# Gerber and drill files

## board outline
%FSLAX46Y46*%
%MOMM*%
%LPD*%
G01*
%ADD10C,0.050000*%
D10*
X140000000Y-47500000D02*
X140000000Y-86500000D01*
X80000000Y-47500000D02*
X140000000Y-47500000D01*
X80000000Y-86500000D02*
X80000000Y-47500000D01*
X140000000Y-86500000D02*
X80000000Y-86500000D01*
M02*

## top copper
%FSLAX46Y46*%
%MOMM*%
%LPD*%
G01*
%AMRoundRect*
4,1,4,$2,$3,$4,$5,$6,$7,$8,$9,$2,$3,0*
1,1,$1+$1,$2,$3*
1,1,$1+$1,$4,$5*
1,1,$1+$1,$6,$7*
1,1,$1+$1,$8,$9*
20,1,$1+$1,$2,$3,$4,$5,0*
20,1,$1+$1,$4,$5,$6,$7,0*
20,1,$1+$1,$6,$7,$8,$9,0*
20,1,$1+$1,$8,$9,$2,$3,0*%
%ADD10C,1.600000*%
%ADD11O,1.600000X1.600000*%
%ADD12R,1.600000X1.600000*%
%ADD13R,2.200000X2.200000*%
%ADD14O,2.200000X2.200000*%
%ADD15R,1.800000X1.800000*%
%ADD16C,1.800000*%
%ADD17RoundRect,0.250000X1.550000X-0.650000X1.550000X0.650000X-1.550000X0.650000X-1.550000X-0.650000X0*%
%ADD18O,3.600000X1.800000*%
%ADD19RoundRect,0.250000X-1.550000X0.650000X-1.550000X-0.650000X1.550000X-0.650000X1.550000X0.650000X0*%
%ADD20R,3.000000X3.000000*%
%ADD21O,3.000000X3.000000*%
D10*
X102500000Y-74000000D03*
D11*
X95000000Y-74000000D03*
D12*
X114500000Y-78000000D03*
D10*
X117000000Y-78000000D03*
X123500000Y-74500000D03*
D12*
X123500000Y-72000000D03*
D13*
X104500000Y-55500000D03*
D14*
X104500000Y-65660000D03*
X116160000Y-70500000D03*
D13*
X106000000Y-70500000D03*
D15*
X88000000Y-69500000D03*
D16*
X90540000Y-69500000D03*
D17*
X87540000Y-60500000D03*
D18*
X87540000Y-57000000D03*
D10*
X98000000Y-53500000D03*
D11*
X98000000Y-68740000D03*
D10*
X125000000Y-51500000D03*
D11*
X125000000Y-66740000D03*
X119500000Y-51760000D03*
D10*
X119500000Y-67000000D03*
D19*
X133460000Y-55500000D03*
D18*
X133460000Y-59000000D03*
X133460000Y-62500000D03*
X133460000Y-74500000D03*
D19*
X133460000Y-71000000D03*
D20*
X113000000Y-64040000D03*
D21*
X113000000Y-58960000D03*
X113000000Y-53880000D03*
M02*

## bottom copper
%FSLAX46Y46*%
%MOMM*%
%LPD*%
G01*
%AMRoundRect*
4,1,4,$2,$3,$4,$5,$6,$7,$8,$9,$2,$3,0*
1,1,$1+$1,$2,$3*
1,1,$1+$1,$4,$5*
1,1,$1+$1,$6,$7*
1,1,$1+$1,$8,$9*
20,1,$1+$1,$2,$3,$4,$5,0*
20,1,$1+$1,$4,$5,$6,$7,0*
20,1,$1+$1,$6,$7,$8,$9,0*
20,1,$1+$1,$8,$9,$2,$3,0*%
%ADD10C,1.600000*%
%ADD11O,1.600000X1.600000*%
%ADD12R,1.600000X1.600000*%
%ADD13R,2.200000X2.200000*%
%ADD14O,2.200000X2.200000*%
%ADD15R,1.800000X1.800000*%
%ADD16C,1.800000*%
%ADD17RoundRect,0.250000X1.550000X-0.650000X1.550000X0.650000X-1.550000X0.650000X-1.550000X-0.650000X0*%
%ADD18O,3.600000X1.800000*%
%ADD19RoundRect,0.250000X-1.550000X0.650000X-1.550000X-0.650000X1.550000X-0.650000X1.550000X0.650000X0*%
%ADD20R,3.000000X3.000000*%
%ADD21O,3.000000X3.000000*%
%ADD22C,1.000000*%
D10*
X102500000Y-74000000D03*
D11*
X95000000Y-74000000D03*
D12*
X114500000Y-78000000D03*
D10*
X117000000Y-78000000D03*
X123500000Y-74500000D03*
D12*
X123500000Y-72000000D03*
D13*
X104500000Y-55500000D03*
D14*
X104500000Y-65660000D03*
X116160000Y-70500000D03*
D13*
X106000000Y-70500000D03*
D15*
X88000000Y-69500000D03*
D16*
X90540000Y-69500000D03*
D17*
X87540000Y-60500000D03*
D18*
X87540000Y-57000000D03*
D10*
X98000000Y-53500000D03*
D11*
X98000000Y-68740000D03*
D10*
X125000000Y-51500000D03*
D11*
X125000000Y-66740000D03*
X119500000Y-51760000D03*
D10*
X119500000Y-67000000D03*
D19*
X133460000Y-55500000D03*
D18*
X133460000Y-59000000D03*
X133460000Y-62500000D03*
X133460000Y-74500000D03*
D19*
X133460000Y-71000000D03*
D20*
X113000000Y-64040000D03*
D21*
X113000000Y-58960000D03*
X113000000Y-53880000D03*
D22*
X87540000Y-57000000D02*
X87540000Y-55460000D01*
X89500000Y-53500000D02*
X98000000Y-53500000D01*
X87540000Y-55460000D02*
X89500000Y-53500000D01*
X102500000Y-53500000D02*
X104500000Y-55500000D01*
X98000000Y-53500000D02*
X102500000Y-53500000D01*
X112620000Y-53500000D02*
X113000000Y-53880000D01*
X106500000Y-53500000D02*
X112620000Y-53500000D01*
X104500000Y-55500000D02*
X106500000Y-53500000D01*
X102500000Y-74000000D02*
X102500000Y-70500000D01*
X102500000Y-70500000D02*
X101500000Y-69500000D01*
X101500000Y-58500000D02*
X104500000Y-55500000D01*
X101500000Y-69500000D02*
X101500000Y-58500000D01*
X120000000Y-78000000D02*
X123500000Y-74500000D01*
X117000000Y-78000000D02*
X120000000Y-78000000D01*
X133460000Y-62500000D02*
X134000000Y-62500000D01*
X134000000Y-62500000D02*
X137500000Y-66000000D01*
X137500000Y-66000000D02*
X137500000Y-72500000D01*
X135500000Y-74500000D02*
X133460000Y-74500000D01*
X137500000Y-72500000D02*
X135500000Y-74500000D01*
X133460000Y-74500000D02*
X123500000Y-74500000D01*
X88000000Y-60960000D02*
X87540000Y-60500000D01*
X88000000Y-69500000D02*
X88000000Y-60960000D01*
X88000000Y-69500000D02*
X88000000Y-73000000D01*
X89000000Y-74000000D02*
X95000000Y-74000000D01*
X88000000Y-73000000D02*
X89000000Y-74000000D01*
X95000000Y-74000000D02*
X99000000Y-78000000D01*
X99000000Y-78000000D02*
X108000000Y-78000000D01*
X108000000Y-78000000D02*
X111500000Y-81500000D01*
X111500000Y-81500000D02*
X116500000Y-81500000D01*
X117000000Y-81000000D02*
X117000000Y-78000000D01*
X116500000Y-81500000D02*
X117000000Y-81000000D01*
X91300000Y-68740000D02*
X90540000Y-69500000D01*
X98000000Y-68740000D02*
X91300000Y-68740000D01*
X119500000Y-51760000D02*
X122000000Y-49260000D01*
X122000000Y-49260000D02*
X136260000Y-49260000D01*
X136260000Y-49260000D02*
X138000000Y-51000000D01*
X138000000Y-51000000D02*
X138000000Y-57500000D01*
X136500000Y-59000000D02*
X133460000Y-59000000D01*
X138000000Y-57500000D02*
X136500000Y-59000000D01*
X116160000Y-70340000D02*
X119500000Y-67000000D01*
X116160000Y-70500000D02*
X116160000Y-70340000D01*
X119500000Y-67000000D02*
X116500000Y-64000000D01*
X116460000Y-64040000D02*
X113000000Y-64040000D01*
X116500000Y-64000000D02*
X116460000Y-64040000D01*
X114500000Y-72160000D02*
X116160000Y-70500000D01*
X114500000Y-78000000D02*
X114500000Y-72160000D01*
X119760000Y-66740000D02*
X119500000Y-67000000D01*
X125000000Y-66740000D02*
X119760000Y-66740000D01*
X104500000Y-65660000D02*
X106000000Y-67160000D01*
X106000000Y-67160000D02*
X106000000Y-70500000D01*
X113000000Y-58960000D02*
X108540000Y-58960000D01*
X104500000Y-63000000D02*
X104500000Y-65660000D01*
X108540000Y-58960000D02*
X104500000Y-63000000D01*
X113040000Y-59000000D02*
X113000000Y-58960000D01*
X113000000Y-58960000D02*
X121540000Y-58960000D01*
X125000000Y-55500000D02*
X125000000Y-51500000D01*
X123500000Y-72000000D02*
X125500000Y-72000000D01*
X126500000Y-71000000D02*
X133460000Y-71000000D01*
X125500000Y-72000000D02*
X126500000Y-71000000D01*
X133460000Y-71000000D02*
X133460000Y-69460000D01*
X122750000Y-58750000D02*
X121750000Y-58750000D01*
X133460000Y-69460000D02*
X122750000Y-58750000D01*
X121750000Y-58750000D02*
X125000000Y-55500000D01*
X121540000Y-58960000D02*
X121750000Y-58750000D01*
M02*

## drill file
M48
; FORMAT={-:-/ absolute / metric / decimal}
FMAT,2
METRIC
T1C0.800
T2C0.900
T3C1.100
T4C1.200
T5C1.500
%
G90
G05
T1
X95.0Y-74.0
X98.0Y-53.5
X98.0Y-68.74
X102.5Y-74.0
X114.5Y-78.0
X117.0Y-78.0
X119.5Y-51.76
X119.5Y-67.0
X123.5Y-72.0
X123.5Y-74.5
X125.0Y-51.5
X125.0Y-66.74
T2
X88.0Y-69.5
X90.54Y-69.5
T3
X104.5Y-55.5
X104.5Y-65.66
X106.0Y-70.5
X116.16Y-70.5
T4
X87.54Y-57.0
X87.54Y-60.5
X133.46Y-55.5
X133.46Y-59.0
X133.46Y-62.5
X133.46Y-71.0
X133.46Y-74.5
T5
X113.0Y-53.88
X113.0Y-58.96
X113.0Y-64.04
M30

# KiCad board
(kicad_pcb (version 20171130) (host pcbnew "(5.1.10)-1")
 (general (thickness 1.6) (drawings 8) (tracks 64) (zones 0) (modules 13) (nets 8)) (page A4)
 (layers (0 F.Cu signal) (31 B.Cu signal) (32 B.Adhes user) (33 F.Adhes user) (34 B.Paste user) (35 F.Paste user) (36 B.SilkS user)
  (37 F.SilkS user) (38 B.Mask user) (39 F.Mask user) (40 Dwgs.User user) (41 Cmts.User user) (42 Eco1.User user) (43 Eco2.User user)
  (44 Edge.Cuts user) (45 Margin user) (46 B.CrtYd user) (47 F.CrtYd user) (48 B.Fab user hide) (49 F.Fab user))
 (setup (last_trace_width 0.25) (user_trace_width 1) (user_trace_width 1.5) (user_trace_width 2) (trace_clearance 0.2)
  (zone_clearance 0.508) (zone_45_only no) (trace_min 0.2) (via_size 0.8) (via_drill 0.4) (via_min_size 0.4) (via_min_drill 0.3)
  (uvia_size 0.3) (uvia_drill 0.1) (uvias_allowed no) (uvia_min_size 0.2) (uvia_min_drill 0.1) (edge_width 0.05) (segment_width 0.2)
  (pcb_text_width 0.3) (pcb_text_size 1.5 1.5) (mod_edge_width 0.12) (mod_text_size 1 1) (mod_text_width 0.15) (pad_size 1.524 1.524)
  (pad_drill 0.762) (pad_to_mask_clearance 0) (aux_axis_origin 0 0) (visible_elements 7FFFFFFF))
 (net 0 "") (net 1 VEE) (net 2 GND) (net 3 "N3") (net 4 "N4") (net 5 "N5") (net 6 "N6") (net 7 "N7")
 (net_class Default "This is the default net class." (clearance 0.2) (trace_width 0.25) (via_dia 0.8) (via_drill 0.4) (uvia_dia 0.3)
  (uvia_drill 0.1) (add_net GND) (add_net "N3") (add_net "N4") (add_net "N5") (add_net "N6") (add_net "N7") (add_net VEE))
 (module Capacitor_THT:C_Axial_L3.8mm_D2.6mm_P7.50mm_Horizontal (layer F.Cu) (at 102.5 74 180)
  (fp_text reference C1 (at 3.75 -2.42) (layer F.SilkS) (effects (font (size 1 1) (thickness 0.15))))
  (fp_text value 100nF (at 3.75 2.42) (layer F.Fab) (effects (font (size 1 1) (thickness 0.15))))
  (pad 1 thru_hole circle (at 0 0 180) (size 1.6 1.6) (drill 0.8) (layers *.Cu *.Mask) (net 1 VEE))
  (pad 2 thru_hole oval (at 7.5 0 180) (size 1.6 1.6) (drill 0.8) (layers *.Cu *.Mask) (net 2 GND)))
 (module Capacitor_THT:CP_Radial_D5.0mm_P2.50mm (layer F.Cu) (at 114.5 78)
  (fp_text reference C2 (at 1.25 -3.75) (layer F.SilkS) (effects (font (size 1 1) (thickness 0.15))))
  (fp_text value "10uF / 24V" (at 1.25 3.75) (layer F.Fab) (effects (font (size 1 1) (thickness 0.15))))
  (pad 1 thru_hole rect (at 0 0) (size 1.6 1.6) (drill 0.8) (layers *.Cu *.Mask) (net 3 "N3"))
  (pad 2 thru_hole circle (at 2.5 0) (size 1.6 1.6) (drill 0.8) (layers *.Cu *.Mask) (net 2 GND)))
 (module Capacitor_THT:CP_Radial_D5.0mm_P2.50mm (layer F.Cu) (at 123.5 72 270)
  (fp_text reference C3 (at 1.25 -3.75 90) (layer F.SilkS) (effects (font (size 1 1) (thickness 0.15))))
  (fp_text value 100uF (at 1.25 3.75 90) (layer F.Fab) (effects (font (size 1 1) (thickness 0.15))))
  (pad 2 thru_hole circle (at 2.5 0 270) (size 1.6 1.6) (drill 0.8) (layers *.Cu *.Mask) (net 2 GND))
  (pad 1 thru_hole rect (at 0 0 270) (size 1.6 1.6) (drill 0.8) (layers *.Cu *.Mask) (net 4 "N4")))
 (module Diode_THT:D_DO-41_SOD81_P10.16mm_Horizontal (layer F.Cu) (at 104.5 55.5 270)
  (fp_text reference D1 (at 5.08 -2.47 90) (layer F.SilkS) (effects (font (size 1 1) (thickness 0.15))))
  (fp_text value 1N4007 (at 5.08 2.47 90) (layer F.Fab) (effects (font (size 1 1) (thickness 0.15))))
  (pad 1 thru_hole rect (at 0 0 270) (size 2.2 2.2) (drill 1.1) (layers *.Cu *.Mask) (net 1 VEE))
  (pad 2 thru_hole oval (at 10.16 0 270) (size 2.2 2.2) (drill 1.1) (layers *.Cu *.Mask) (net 4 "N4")))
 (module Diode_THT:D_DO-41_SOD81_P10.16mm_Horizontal (layer F.Cu) (at 106 70.5)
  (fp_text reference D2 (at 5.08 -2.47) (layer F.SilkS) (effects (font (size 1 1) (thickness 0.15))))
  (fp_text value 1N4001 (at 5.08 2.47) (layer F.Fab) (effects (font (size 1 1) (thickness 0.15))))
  (pad 2 thru_hole oval (at 10.16 0) (size 2.2 2.2) (drill 1.1) (layers *.Cu *.Mask) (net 3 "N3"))
  (pad 1 thru_hole rect (at 0 0) (size 2.2 2.2) (drill 1.1) (layers *.Cu *.Mask) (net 4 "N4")))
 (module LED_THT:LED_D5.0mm (layer F.Cu) (at 88 69.5)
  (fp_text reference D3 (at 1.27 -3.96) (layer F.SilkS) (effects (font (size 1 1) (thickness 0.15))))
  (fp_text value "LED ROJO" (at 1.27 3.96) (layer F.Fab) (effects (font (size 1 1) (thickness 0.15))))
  (pad 1 thru_hole rect (at 0 0) (size 1.8 1.8) (drill 0.9) (layers *.Cu *.Mask) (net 2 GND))
  (pad 2 thru_hole circle (at 2.54 0) (size 1.8 1.8) (drill 0.9) (layers *.Cu *.Mask) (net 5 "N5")))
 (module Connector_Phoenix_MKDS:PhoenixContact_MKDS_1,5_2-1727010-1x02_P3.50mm (layer F.Cu) (at 85 60.5 90)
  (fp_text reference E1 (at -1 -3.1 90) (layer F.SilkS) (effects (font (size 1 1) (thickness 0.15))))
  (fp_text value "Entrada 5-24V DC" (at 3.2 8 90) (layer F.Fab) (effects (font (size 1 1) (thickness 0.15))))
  (pad 1 thru_hole roundrect (at 0 2.54 90) (size 1.8 3.6) (drill 1.2) (layers *.Cu *.Mask) (roundrect_rratio 0.138889) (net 2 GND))
  (pad 2 thru_hole oval (at 3.5 2.54 90) (size 1.8 3.6) (drill 1.2) (layers *.Cu *.Mask) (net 1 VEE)))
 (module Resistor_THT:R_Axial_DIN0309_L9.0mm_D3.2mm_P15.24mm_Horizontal (layer F.Cu) (at 98 53.5 270)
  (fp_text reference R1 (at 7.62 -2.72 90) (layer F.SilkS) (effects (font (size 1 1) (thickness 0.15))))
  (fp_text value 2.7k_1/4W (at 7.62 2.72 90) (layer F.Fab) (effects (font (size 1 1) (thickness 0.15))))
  (pad 1 thru_hole circle (at 0 0 270) (size 1.6 1.6) (drill 0.8) (layers *.Cu *.Mask) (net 1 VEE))
  (pad 2 thru_hole oval (at 15.24 0 270) (size 1.6 1.6) (drill 0.8) (layers *.Cu *.Mask) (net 5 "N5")))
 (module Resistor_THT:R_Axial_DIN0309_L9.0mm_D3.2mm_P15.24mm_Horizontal (layer F.Cu) (at 125 51.5 270)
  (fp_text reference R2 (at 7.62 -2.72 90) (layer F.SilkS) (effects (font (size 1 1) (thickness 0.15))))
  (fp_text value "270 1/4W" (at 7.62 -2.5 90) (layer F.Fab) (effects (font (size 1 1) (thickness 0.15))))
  (pad 1 thru_hole circle (at 0 0 270) (size 1.6 1.6) (drill 0.8) (layers *.Cu *.Mask) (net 4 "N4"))
  (pad 2 thru_hole oval (at 15.24 0 270) (size 1.6 1.6) (drill 0.8) (layers *.Cu *.Mask) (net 3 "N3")))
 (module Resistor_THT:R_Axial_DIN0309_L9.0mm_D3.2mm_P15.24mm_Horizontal (layer F.Cu) (at 119.5 67 90)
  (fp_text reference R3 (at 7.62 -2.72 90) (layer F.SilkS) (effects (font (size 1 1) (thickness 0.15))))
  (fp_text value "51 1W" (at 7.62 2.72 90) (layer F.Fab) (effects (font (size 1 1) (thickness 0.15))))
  (pad 2 thru_hole oval (at 15.24 0 90) (size 1.6 1.6) (drill 0.8) (layers *.Cu *.Mask) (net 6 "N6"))
  (pad 1 thru_hole circle (at 0 0 90) (size 1.6 1.6) (drill 0.8) (layers *.Cu *.Mask) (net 3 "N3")))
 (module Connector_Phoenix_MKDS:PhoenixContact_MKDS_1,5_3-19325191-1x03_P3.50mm (layer F.Cu) (at 136 55.5 270)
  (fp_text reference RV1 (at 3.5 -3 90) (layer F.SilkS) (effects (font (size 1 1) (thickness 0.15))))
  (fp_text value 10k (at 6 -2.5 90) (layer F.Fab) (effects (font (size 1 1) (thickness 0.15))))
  (pad 1 thru_hole roundrect (at 0 2.54 270) (size 1.8 3.6) (drill 1.2) (layers *.Cu *.Mask) (roundrect_rratio 0.138889) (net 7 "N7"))
  (pad 2 thru_hole oval (at 3.5 2.54 270) (size 1.8 3.6) (drill 1.2) (layers *.Cu *.Mask) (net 6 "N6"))
  (pad 3 thru_hole oval (at 7 2.54 270) (size 1.8 3.6) (drill 1.2) (layers *.Cu *.Mask) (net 2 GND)))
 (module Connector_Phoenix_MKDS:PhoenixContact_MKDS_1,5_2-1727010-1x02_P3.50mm (layer F.Cu) (at 136 71 270)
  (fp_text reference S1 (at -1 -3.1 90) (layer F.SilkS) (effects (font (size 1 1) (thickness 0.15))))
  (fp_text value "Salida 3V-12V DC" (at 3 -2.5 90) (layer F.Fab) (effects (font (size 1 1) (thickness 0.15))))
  (pad 2 thru_hole oval (at 3.5 2.54 270) (size 1.8 3.6) (drill 1.2) (layers *.Cu *.Mask) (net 2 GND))
  (pad 1 thru_hole roundrect (at 0 2.54 270) (size 1.8 3.6) (drill 1.2) (layers *.Cu *.Mask) (roundrect_rratio 0.138889) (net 4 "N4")))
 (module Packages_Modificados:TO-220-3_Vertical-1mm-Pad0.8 (layer F.Cu) (at 113 61.5 90)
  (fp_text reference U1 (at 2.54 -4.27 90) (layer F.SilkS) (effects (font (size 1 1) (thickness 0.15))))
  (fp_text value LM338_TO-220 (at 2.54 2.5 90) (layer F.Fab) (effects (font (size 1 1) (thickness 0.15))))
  (pad 1 thru_hole rect (at -2.54 0 90) (size 3 3) (drill 1.5) (layers *.Cu *.Mask) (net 3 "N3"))
  (pad 2 thru_hole oval (at 2.54 0 90) (size 3 3) (drill 1.5) (layers *.Cu *.Mask) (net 4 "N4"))
  (pad 3 thru_hole oval (at 7.62 0 90) (size 3 3) (drill 1.5) (layers *.Cu *.Mask) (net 1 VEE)))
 (gr_line (start 140 47.5) (end 140 86.5) (layer Edge.Cuts) (width 0.05))
 (gr_line (start 80 47.5) (end 140 47.5) (layer Edge.Cuts) (width 0.05))
 (gr_line (start 80 86.5) (end 80 47.5) (layer Edge.Cuts) (width 0.05))
 (gr_line (start 140 86.5) (end 80 86.5) (layer Edge.Cuts) (width 0.05))
 (segment (start 87.54 57) (end 87.54 55.46) (width 1) (layer B.Cu) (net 1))
 (segment (start 89.5 53.5) (end 98 53.5) (width 1) (layer B.Cu) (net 1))
 (segment (start 87.54 55.46) (end 89.5 53.5) (width 1) (layer B.Cu) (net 1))
 (segment (start 102.5 53.5) (end 104.5 55.5) (width 1) (layer B.Cu) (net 1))
 (segment (start 98 53.5) (end 102.5 53.5) (width 1) (layer B.Cu) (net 1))
 (segment (start 112.62 53.5) (end 113 53.88) (width 1) (layer B.Cu) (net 1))
 (segment (start 106.5 53.5) (end 112.62 53.5) (width 1) (layer B.Cu) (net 1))
 (segment (start 104.5 55.5) (end 106.5 53.5) (width 1) (layer B.Cu) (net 1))
 (segment (start 102.5 74) (end 102.5 70.5) (width 1) (layer B.Cu) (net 1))
 (segment (start 102.5 70.5) (end 101.5 69.5) (width 1) (layer B.Cu) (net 1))
 (segment (start 101.5 58.5) (end 104.5 55.5) (width 1) (layer B.Cu) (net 1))
 (segment (start 101.5 69.5) (end 101.5 58.5) (width 1) (layer B.Cu) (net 1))
 (segment (start 120 78) (end 123.5 74.5) (width 1) (layer B.Cu) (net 2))
 (segment (start 117 78) (end 120 78) (width 1) (layer B.Cu) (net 2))
 (segment (start 133.46 62.5) (end 134 62.5) (width 1) (layer B.Cu) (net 2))
 (segment (start 134 62.5) (end 137.5 66) (width 1) (layer B.Cu) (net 2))
 (segment (start 137.5 66) (end 137.5 72.5) (width 1) (layer B.Cu) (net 2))
 (segment (start 135.5 74.5) (end 133.46 74.5) (width 1) (layer B.Cu) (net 2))
 (segment (start 137.5 72.5) (end 135.5 74.5) (width 1) (layer B.Cu) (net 2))
 (segment (start 133.46 74.5) (end 123.5 74.5) (width 1) (layer B.Cu) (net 2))
 (segment (start 88 60.96) (end 87.54 60.5) (width 1) (layer B.Cu) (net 2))
 (segment (start 88 69.5) (end 88 60.96) (width 1) (layer B.Cu) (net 2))
 (segment (start 88 69.5) (end 88 73) (width 1) (layer B.Cu) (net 2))
 (segment (start 89 74) (end 95 74) (width 1) (layer B.Cu) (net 2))
 (segment (start 88 73) (end 89 74) (width 1) (layer B.Cu) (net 2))
 (segment (start 95 74) (end 99 78) (width 1) (layer B.Cu) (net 2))
 (segment (start 99 78) (end 108 78) (width 1) (layer B.Cu) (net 2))
 (segment (start 108 78) (end 111.5 81.5) (width 1) (layer B.Cu) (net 2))
 (segment (start 111.5 81.5) (end 116.5 81.5) (width 1) (layer B.Cu) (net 2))
 (segment (start 117 81) (end 117 78) (width 1) (layer B.Cu) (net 2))
 (segment (start 116.5 81.5) (end 117 81) (width 1) (layer B.Cu) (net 2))
 (segment (start 91.3 68.74) (end 90.54 69.5) (width 1) (layer B.Cu) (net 5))
 (segment (start 98 68.74) (end 91.3 68.74) (width 1) (layer B.Cu) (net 5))
 (segment (start 119.5 51.76) (end 122 49.26) (width 1) (layer B.Cu) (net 6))
 (segment (start 122 49.26) (end 136.26 49.26) (width 1) (layer B.Cu) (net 6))
 (segment (start 136.26 49.26) (end 138 51) (width 1) (layer B.Cu) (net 6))
 (segment (start 138 51) (end 138 57.5) (width 1) (layer B.Cu) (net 6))
 (segment (start 136.5 59) (end 133.46 59) (width 1) (layer B.Cu) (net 6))
 (segment (start 138 57.5) (end 136.5 59) (width 1) (layer B.Cu) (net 6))
 (segment (start 116.16 70.34) (end 119.5 67) (width 1) (layer B.Cu) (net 3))
 (segment (start 116.16 70.5) (end 116.16 70.34) (width 1) (layer B.Cu) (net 3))
 (segment (start 119.5 67) (end 116.5 64) (width 1) (layer B.Cu) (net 3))
 (segment (start 116.46 64.04) (end 113 64.04) (width 1) (layer B.Cu) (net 3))
 (segment (start 116.5 64) (end 116.46 64.04) (width 1) (layer B.Cu) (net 3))
 (segment (start 114.5 72.16) (end 116.16 70.5) (width 1) (layer B.Cu) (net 3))
 (segment (start 114.5 78) (end 114.5 72.16) (width 1) (layer B.Cu) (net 3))
 (segment (start 119.76 66.74) (end 119.5 67) (width 1) (layer B.Cu) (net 3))
 (segment (start 125 66.74) (end 119.76 66.74) (width 1) (layer B.Cu) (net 3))
 (segment (start 104.5 65.66) (end 106 67.16) (width 1) (layer B.Cu) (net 4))
 (segment (start 106 67.16) (end 106 70.5) (width 1) (layer B.Cu) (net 4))
 (segment (start 113 58.96) (end 108.54 58.96) (width 1) (layer B.Cu) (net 4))
 (segment (start 104.5 63) (end 104.5 65.66) (width 1) (layer B.Cu) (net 4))
 (segment (start 108.54 58.96) (end 104.5 63) (width 1) (layer B.Cu) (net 4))
 (segment (start 113.04 59) (end 113 58.96) (width 1) (layer B.Cu) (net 4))
 (segment (start 113 58.96) (end 121.54 58.96) (width 1) (layer B.Cu) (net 4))
 (segment (start 125 55.5) (end 125 51.5) (width 1) (layer B.Cu) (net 4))
 (segment (start 123.5 72) (end 125.5 72) (width 1) (layer B.Cu) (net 4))
 (segment (start 126.5 71) (end 133.46 71) (width 1) (layer B.Cu) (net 4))
 (segment (start 125.5 72) (end 126.5 71) (width 1) (layer B.Cu) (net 4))
 (segment (start 133.46 71) (end 133.46 69.46) (width 1) (layer B.Cu) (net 4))
 (segment (start 122.75 58.75) (end 121.75 58.75) (width 1) (layer B.Cu) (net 4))
 (segment (start 133.46 69.46) (end 122.75 58.75) (width 1) (layer B.Cu) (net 4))
 (segment (start 121.75 58.75) (end 125 55.5) (width 1) (layer B.Cu) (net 4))
 (segment (start 121.54 58.96) (end 121.75 58.75) (width 1) (layer B.Cu) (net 4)))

